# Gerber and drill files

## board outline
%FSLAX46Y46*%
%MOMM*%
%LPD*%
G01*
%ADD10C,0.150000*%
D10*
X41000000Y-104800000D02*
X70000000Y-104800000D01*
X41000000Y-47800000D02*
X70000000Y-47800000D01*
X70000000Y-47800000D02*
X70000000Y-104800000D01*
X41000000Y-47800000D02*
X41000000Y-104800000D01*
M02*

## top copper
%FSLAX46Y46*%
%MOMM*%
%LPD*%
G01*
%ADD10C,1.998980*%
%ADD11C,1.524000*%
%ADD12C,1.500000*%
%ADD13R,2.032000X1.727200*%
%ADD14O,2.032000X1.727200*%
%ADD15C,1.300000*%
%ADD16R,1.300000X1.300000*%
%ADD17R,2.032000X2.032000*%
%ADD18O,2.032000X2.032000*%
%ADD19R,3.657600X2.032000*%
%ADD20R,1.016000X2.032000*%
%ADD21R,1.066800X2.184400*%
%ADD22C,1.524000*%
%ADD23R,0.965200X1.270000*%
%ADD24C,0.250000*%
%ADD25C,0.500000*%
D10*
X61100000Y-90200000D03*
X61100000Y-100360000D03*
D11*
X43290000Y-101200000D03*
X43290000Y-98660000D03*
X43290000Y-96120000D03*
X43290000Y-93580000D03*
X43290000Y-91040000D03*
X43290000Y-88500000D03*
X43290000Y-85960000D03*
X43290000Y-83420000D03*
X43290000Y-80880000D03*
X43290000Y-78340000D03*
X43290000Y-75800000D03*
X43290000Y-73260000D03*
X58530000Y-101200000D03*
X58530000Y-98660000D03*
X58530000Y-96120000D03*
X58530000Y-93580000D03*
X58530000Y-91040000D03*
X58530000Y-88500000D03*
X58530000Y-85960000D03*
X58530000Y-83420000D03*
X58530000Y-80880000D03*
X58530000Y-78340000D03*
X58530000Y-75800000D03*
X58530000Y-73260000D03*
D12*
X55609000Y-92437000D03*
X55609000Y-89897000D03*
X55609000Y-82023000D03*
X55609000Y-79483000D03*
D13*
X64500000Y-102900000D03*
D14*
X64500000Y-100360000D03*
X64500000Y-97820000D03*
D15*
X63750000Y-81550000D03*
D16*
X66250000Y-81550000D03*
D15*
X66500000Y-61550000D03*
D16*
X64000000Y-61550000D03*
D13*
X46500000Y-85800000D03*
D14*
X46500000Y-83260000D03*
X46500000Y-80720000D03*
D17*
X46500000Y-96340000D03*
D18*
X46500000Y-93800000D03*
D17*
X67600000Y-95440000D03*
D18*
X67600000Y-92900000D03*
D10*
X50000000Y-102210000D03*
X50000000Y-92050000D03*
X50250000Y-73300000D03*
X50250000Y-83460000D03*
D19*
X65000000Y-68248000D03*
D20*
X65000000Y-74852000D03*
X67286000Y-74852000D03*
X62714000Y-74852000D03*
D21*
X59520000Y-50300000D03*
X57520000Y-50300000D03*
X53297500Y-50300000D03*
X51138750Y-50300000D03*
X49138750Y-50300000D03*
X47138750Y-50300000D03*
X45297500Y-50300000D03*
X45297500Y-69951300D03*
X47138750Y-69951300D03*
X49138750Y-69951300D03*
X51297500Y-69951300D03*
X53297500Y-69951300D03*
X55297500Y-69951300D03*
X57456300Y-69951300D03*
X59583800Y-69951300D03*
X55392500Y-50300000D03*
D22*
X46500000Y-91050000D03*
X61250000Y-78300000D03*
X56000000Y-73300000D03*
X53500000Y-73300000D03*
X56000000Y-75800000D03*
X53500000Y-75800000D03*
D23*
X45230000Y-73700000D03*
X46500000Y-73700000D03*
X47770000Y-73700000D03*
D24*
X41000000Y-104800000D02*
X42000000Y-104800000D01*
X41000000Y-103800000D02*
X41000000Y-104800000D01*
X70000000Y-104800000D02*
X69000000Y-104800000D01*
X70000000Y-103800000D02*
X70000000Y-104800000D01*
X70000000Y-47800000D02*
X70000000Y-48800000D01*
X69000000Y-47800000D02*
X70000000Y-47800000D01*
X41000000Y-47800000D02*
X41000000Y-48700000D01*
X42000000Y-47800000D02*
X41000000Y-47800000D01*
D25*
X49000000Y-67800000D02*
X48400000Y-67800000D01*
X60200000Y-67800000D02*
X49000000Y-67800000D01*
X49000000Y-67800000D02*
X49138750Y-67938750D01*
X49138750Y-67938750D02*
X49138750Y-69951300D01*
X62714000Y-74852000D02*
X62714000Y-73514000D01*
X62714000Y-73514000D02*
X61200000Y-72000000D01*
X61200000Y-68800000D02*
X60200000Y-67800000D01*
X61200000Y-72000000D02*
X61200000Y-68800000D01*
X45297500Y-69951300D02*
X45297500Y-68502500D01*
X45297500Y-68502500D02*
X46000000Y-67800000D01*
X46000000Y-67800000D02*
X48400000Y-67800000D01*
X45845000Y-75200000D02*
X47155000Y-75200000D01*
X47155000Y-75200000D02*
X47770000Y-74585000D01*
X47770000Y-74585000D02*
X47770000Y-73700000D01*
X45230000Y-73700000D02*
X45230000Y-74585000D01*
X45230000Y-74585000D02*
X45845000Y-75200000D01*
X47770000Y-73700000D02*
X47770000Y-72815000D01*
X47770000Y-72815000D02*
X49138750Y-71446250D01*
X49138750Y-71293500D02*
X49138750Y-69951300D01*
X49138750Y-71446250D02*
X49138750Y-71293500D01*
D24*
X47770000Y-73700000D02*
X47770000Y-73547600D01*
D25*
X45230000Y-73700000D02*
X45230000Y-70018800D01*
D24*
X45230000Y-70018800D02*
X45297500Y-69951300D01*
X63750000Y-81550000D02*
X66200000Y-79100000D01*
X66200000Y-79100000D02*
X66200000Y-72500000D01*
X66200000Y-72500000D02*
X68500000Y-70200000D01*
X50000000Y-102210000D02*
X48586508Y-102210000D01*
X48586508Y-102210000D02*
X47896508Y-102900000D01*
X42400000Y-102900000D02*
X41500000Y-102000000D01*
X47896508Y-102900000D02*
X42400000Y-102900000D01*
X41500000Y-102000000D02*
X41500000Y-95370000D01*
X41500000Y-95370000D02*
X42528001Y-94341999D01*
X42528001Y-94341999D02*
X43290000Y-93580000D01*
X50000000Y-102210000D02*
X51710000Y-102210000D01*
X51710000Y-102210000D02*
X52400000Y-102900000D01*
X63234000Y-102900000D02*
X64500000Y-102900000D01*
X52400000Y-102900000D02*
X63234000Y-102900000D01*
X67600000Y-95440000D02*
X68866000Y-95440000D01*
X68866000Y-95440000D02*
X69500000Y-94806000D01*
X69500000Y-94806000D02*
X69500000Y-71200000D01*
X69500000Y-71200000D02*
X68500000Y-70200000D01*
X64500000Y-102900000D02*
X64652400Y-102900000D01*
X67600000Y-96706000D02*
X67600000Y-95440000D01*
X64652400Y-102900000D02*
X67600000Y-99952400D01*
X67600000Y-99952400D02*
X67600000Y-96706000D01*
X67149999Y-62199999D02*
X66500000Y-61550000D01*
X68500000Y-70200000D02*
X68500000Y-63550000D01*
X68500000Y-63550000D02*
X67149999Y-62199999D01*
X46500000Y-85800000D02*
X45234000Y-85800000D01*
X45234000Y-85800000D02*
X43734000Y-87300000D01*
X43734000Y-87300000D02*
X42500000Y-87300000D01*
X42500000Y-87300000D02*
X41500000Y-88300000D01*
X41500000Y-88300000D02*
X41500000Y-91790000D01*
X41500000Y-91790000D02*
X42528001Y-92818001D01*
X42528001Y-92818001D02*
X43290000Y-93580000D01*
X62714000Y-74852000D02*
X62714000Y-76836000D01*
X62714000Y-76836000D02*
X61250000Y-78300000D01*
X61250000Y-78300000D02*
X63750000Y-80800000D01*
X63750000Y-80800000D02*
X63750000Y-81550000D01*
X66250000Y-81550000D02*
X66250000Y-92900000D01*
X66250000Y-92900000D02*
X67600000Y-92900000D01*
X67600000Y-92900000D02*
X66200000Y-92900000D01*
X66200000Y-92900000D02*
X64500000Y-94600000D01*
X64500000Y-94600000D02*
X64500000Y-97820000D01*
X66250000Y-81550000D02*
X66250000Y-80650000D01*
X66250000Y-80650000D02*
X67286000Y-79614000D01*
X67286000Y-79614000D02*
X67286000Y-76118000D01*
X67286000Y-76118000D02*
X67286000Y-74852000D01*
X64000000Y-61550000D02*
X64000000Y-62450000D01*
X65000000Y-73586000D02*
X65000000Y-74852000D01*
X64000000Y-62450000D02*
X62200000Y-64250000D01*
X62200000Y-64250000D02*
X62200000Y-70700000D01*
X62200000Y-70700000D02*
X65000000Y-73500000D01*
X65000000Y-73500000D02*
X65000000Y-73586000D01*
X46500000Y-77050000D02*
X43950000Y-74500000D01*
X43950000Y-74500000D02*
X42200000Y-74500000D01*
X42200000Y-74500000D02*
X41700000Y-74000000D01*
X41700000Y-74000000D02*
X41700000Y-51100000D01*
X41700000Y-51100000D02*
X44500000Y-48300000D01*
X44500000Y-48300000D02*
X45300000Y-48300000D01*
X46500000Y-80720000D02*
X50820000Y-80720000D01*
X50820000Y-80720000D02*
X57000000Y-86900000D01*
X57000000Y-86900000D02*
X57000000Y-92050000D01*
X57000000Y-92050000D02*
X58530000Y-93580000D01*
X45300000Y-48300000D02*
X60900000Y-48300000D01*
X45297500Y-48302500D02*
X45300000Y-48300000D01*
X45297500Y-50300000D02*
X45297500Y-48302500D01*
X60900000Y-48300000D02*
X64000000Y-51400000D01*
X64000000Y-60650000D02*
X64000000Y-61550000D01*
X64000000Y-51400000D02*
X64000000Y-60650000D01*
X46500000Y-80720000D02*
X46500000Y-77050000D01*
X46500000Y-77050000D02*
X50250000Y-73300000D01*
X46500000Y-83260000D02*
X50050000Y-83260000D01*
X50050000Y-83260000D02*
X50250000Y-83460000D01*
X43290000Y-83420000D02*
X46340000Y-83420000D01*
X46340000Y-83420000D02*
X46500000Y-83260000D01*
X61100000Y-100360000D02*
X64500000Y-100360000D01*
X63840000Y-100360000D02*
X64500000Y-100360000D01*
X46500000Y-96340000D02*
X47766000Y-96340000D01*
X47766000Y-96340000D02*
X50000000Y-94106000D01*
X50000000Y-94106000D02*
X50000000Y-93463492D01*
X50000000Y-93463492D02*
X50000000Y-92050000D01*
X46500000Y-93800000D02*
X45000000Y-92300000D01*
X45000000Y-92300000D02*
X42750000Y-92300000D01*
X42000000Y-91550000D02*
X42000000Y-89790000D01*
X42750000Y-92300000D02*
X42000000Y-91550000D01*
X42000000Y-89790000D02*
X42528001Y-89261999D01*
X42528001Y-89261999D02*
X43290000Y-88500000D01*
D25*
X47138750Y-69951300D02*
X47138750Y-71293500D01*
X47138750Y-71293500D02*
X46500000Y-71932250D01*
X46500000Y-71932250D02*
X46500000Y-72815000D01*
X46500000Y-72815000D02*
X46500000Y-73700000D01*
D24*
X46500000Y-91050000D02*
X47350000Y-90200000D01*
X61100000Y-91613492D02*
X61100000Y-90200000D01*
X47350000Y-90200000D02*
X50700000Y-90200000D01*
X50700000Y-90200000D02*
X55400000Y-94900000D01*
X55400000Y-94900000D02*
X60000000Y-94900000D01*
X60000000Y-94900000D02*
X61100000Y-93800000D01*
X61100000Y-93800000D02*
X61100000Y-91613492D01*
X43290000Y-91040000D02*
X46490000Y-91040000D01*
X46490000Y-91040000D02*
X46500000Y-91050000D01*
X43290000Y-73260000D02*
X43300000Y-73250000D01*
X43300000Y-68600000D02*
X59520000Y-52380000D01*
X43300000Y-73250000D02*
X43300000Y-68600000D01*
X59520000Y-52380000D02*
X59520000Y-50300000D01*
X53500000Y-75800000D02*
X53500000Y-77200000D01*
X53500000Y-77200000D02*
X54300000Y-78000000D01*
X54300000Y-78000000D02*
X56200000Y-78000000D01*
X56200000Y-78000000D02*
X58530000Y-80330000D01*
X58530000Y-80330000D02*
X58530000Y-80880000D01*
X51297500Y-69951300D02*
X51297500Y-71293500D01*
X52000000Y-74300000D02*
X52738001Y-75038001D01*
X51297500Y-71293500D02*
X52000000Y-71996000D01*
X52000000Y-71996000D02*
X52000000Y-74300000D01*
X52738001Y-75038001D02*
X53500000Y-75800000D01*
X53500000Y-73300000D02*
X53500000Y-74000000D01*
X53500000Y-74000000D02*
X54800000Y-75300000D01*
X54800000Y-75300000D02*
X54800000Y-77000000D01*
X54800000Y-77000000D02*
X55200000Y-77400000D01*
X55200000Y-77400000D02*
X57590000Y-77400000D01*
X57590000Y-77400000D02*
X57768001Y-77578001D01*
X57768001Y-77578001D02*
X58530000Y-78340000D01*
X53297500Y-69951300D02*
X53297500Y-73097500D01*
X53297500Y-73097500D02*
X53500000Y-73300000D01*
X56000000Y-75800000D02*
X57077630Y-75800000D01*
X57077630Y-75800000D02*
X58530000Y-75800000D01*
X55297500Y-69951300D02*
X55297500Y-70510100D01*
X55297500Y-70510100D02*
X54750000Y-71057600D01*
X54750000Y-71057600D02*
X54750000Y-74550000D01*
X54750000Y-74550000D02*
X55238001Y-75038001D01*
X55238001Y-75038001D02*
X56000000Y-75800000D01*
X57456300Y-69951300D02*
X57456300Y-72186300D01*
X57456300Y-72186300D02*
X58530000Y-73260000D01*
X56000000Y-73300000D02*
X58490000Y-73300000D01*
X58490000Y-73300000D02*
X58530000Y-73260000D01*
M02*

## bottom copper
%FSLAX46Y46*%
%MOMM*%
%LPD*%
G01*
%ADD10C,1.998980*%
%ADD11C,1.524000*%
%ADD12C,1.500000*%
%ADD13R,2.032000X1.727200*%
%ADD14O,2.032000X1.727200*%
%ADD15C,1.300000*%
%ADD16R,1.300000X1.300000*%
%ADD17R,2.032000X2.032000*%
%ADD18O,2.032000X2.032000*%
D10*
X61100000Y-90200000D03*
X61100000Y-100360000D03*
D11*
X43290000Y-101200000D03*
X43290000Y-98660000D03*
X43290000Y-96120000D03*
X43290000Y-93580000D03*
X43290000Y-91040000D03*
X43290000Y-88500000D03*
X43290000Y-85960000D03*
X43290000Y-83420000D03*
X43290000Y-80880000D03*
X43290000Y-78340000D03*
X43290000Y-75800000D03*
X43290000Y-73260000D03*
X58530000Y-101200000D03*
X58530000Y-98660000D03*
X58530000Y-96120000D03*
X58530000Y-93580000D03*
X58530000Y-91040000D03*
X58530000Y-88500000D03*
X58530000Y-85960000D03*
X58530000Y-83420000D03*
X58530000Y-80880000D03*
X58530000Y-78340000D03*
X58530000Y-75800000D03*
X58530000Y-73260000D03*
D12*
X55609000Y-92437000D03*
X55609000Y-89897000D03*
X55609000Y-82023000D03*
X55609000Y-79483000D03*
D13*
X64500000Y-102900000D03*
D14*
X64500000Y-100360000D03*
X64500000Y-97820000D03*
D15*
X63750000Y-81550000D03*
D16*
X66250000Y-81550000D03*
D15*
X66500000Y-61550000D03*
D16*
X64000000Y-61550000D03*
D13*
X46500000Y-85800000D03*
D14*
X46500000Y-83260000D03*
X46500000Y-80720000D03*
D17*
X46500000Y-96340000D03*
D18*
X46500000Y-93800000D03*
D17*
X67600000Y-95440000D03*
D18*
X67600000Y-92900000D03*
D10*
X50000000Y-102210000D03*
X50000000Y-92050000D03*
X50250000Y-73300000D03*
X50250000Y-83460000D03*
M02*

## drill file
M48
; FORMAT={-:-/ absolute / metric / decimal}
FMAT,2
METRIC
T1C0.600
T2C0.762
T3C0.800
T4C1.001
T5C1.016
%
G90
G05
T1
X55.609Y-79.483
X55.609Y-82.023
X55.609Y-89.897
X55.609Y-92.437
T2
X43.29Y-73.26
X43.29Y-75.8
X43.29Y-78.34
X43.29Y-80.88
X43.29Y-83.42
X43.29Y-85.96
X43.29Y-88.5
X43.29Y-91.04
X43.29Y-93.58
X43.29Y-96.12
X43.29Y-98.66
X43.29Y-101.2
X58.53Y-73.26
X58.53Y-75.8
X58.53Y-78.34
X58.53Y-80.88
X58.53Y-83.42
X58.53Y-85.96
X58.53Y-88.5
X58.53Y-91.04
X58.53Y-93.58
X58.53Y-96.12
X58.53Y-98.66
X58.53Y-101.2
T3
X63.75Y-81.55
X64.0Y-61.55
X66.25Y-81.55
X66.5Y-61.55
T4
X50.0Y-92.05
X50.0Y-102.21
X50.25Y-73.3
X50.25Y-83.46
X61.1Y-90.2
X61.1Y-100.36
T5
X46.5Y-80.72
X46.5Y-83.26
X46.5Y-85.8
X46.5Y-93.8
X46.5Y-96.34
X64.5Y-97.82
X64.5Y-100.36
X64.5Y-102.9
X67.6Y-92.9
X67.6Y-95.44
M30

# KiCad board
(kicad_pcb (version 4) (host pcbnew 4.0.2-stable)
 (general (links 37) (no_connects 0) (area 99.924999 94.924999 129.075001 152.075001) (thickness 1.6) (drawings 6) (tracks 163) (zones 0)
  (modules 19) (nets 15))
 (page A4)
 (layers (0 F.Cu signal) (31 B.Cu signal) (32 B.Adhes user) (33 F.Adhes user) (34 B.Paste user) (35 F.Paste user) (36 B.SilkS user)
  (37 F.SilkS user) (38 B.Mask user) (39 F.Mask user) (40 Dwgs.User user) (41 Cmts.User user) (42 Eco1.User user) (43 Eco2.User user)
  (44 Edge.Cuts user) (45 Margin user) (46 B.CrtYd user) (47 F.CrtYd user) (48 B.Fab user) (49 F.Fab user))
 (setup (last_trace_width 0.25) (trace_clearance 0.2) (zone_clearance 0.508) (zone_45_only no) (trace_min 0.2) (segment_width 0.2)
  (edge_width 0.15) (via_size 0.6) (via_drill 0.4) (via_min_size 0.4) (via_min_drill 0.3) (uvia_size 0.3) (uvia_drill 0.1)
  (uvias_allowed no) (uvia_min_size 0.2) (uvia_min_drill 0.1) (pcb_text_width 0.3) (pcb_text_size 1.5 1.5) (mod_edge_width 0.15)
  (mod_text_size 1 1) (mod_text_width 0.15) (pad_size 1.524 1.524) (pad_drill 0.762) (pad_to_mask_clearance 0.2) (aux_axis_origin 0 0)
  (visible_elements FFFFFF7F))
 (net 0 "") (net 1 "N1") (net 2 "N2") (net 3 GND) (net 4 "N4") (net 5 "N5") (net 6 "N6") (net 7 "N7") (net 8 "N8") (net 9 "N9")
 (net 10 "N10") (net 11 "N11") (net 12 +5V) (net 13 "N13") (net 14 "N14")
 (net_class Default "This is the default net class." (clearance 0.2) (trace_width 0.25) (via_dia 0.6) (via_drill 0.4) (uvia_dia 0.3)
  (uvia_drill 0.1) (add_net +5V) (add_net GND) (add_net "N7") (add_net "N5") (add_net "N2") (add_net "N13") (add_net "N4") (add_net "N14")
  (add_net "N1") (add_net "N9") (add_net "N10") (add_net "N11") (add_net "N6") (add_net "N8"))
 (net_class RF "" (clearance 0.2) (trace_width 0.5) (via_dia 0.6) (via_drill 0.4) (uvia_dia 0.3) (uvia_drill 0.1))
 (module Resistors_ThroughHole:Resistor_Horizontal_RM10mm (layer F.Cu) (at 61.1 90.2 270)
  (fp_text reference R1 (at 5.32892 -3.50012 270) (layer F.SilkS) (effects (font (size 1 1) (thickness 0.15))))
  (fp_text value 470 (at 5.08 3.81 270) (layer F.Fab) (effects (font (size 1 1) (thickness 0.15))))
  (pad 1 thru_hole circle (at 0 0 270) (size 1.99898 1.99898) (drill 1.00076) (layers *.Cu *.SilkS *.Mask) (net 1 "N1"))
  (pad 2 thru_hole circle (at 10.16 0 270) (size 1.99898 1.99898) (drill 1.00076) (layers *.Cu *.SilkS *.Mask) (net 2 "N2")))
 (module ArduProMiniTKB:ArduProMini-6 (layer B.Cu) (at 40.75 107.55)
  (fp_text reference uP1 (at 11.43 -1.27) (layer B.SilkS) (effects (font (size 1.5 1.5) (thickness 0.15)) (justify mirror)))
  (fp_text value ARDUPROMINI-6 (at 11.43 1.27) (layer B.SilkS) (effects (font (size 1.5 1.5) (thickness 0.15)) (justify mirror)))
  (pad 7 thru_hole circle (at 2.54 -6.35) (size 1.524 1.524) (drill 0.762) (layers *.Cu *.Mask B.SilkS))
  (pad 8 thru_hole circle (at 2.54 -8.89) (size 1.524 1.524) (drill 0.762) (layers *.Cu *.Mask B.SilkS))
  (pad 9 thru_hole circle (at 2.54 -11.43) (size 1.524 1.524) (drill 0.762) (layers *.Cu *.Mask B.SilkS))
  (pad 10 thru_hole circle (at 2.54 -13.97) (size 1.524 1.524) (drill 0.762) (layers *.Cu *.Mask B.SilkS) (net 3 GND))
  (pad 11 thru_hole circle (at 2.54 -16.51) (size 1.524 1.524) (drill 0.762) (layers *.Cu *.Mask B.SilkS) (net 1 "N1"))
  (pad 12 thru_hole circle (at 2.54 -19.05) (size 1.524 1.524) (drill 0.762) (layers *.Cu *.Mask B.SilkS) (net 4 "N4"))
  (pad 13 thru_hole circle (at 2.54 -21.59) (size 1.524 1.524) (drill 0.762) (layers *.Cu *.Mask B.SilkS))
  (pad 14 thru_hole circle (at 2.54 -24.13) (size 1.524 1.524) (drill 0.762) (layers *.Cu *.Mask B.SilkS) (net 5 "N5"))
  (pad 15 thru_hole circle (at 2.54 -26.67) (size 1.524 1.524) (drill 0.762) (layers *.Cu *.Mask B.SilkS))
  (pad 16 thru_hole circle (at 2.54 -29.21) (size 1.524 1.524) (drill 0.762) (layers *.Cu *.Mask B.SilkS))
  (pad 17 thru_hole circle (at 2.54 -31.75) (size 1.524 1.524) (drill 0.762) (layers *.Cu *.Mask B.SilkS))
  (pad 18 thru_hole circle (at 2.54 -34.29) (size 1.524 1.524) (drill 0.762) (layers *.Cu *.Mask B.SilkS) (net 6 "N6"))
  (pad 19 thru_hole circle (at 17.78 -6.35) (size 1.524 1.524) (drill 0.762) (layers *.Cu *.Mask B.SilkS))
  (pad 20 thru_hole circle (at 17.78 -8.89) (size 1.524 1.524) (drill 0.762) (layers *.Cu *.Mask B.SilkS))
  (pad 21 thru_hole circle (at 17.78 -11.43) (size 1.524 1.524) (drill 0.762) (layers *.Cu *.Mask B.SilkS))
  (pad 22 thru_hole circle (at 17.78 -13.97) (size 1.524 1.524) (drill 0.762) (layers *.Cu *.Mask B.SilkS) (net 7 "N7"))
  (pad 23 thru_hole circle (at 17.78 -16.51) (size 1.524 1.524) (drill 0.762) (layers *.Cu *.Mask B.SilkS))
  (pad 24 thru_hole circle (at 17.78 -19.05) (size 1.524 1.524) (drill 0.762) (layers *.Cu *.Mask B.SilkS))
  (pad 25 thru_hole circle (at 17.78 -21.59) (size 1.524 1.524) (drill 0.762) (layers *.Cu *.Mask B.SilkS))
  (pad 26 thru_hole circle (at 17.78 -24.13) (size 1.524 1.524) (drill 0.762) (layers *.Cu *.Mask B.SilkS))
  (pad 27 thru_hole circle (at 17.78 -26.67) (size 1.524 1.524) (drill 0.762) (layers *.Cu *.Mask B.SilkS) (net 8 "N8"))
  (pad 28 thru_hole circle (at 17.78 -29.21) (size 1.524 1.524) (drill 0.762) (layers *.Cu *.Mask B.SilkS) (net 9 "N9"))
  (pad 29 thru_hole circle (at 17.78 -31.75) (size 1.524 1.524) (drill 0.762) (layers *.Cu *.Mask B.SilkS) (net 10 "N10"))
  (pad 30 thru_hole circle (at 17.78 -34.29) (size 1.524 1.524) (drill 0.762) (layers *.Cu *.Mask B.SilkS) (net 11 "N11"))
  (pad 31 thru_hole circle (at 14.859 -15.113) (size 1.5 1.5) (drill 0.6) (layers *.Cu *.Mask B.SilkS))
  (pad 32 thru_hole circle (at 14.859 -17.653) (size 1.5 1.5) (drill 0.6) (layers *.Cu *.Mask B.SilkS))
  (pad 34 thru_hole circle (at 14.859 -25.527) (size 1.5 1.5) (drill 0.6) (layers *.Cu *.Mask B.SilkS))
  (pad 35 thru_hole circle (at 14.859 -28.067) (size 1.5 1.5) (drill 0.6) (layers *.Cu *.Mask B.SilkS)))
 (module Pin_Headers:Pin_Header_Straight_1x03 (layer F.Cu) (at 64.5 102.9 180)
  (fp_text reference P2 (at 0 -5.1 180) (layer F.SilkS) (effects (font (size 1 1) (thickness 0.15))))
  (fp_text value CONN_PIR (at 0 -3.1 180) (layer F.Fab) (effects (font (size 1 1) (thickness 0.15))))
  (pad 1 thru_hole rect (at 0 0 180) (size 2.032 1.7272) (drill 1.016) (layers *.Cu *.Mask F.SilkS) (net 3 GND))
  (pad 2 thru_hole oval (at 0 2.54 180) (size 2.032 1.7272) (drill 1.016) (layers *.Cu *.Mask F.SilkS) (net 2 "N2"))
  (pad 3 thru_hole oval (at 0 5.08 180) (size 2.032 1.7272) (drill 1.016) (layers *.Cu *.Mask F.SilkS) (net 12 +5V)))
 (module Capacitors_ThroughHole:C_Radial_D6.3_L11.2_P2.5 (layer F.Cu) (at 66.25 81.55 180)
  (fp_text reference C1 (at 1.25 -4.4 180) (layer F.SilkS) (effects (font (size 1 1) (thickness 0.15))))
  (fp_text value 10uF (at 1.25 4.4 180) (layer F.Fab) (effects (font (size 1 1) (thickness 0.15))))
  (pad 2 thru_hole circle (at 2.5 0 180) (size 1.3 1.3) (drill 0.8) (layers *.Cu *.Mask F.SilkS) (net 3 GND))
  (pad 1 thru_hole rect (at 0 0 180) (size 1.3 1.3) (drill 0.8) (layers *.Cu *.Mask F.SilkS) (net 12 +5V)))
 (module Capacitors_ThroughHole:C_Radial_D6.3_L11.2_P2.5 (layer F.Cu) (at 64 61.55)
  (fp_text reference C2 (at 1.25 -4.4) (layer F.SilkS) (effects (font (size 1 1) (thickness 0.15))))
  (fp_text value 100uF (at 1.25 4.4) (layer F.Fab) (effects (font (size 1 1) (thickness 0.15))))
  (pad 2 thru_hole circle (at 2.5 0) (size 1.3 1.3) (drill 0.8) (layers *.Cu *.Mask F.SilkS) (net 3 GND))
  (pad 1 thru_hole rect (at 0 0) (size 1.3 1.3) (drill 0.8) (layers *.Cu *.Mask F.SilkS) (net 7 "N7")))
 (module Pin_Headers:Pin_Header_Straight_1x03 (layer F.Cu) (at 46.5 85.8 180)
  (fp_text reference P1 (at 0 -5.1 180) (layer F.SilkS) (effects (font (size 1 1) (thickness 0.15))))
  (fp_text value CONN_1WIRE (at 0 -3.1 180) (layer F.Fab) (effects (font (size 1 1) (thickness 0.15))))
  (pad 1 thru_hole rect (at 0 0 180) (size 2.032 1.7272) (drill 1.016) (layers *.Cu *.Mask F.SilkS) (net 3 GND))
  (pad 2 thru_hole oval (at 0 2.54 180) (size 2.032 1.7272) (drill 1.016) (layers *.Cu *.Mask F.SilkS) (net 5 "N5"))
  (pad 3 thru_hole oval (at 0 5.08 180) (size 2.032 1.7272) (drill 1.016) (layers *.Cu *.Mask F.SilkS) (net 7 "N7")))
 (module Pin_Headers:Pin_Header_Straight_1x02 (layer F.Cu) (at 46.5 96.34 180)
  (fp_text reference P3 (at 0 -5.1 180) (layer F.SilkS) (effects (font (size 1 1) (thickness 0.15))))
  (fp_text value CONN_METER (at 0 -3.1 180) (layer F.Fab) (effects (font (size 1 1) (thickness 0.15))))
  (pad 1 thru_hole rect (at 0 0 180) (size 2.032 2.032) (drill 1.016) (layers *.Cu *.Mask F.SilkS) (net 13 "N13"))
  (pad 2 thru_hole oval (at 0 2.54 180) (size 2.032 2.032) (drill 1.016) (layers *.Cu *.Mask F.SilkS) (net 4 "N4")))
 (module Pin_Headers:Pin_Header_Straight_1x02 (layer F.Cu) (at 67.6 95.44 180)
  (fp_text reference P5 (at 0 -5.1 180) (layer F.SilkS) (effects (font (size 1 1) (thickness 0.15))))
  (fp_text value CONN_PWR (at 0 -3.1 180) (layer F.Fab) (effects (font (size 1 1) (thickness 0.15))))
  (pad 1 thru_hole rect (at 0 0 180) (size 2.032 2.032) (drill 1.016) (layers *.Cu *.Mask F.SilkS) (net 3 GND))
  (pad 2 thru_hole oval (at 0 2.54 180) (size 2.032 2.032) (drill 1.016) (layers *.Cu *.Mask F.SilkS) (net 12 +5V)))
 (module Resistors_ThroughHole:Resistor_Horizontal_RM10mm (layer F.Cu) (at 50 102.21 90)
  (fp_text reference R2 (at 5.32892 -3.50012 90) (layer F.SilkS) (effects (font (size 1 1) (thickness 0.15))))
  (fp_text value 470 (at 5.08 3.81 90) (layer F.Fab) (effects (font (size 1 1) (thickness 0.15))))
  (pad 1 thru_hole circle (at 0 0 90) (size 1.99898 1.99898) (drill 1.00076) (layers *.Cu *.SilkS *.Mask) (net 3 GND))
  (pad 2 thru_hole circle (at 10.16 0 90) (size 1.99898 1.99898) (drill 1.00076) (layers *.Cu *.SilkS *.Mask) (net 13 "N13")))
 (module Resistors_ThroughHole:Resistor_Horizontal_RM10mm (layer F.Cu) (at 50.25 73.3 270)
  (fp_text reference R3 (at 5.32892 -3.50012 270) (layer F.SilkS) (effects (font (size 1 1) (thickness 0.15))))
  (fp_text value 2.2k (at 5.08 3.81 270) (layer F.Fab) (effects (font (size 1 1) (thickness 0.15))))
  (pad 1 thru_hole circle (at 0 0 270) (size 1.99898 1.99898) (drill 1.00076) (layers *.Cu *.SilkS *.Mask) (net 7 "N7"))
  (pad 2 thru_hole circle (at 10.16 0 270) (size 1.99898 1.99898) (drill 1.00076) (layers *.Cu *.SilkS *.Mask) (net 5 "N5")))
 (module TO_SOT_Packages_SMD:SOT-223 (layer F.Cu) (at 65 71.55)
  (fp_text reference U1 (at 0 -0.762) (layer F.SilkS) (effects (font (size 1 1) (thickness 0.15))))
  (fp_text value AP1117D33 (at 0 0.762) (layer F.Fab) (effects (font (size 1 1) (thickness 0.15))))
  (pad 4 smd rect (at 0 -3.302) (size 3.6576 2.032) (layers F.Cu F.Paste F.Mask))
  (pad 2 smd rect (at 0 3.302) (size 1.016 2.032) (layers F.Cu F.Paste F.Mask) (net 7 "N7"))
  (pad 3 smd rect (at 2.286 3.302) (size 1.016 2.032) (layers F.Cu F.Paste F.Mask) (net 12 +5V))
  (pad 1 smd rect (at -2.286 3.302) (size 1.016 2.032) (layers F.Cu F.Paste F.Mask) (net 3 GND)))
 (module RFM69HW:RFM (layer F.Cu) (at 44.25 50.3 270) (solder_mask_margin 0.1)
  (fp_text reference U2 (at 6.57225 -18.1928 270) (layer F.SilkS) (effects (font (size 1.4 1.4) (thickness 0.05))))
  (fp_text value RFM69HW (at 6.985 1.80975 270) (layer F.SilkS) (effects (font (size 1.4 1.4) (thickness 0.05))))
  (pad RESE smd rect (at 0 -15.27 270) (size 2.1844 1.0668) (layers F.Cu F.Paste F.Mask) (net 6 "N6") (solder_mask_margin 0.2))
  (pad DIO0 smd rect (at 0 -13.27 270) (size 2.1844 1.0668) (layers F.Cu F.Paste F.Mask) (solder_mask_margin 0.2))
  (pad DIO2 smd rect (at 0 -9.0475 270) (size 2.1844 1.0668) (layers F.Cu F.Paste F.Mask) (solder_mask_margin 0.2))
  (pad DIO3 smd rect (at 0 -6.88875 270) (size 2.1844 1.0668) (layers F.Cu F.Paste F.Mask) (solder_mask_margin 0.2))
  (pad DIO4 smd rect (at 0 -4.88875 270) (size 2.1844 1.0668) (layers F.Cu F.Paste F.Mask) (solder_mask_margin 0.2))
  (pad DIO5 smd rect (at 0 -2.88875 270) (size 2.1844 1.0668) (layers F.Cu F.Paste F.Mask) (solder_mask_margin 0.2))
  (pad VCC smd rect (at 0 -1.0475 270) (size 2.1844 1.0668) (layers F.Cu F.Paste F.Mask) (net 7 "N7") (solder_mask_margin 0.2))
  (pad GNDB smd rect (at 19.6513 -1.0475 270) (size 2.1844 1.0668) (layers F.Cu F.Paste F.Mask) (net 3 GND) (solder_mask_margin 0.2))
  (pad ANT smd rect (at 19.6513 -2.88875 270) (size 2.1844 1.0668) (layers F.Cu F.Paste F.Mask) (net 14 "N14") (solder_mask_margin 0.2))
  (pad GNDA smd rect (at 19.6513 -4.88875 270) (size 2.1844 1.0668) (layers F.Cu F.Paste F.Mask) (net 3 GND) (solder_mask_margin 0.2))
  (pad SCK smd rect (at 19.6513 -7.0475 270) (size 2.1844 1.0668) (layers F.Cu F.Paste F.Mask) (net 8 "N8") (solder_mask_margin 0.2))
  (pad MISO smd rect (at 19.6513 -9.0475 270) (size 2.1844 1.0668) (layers F.Cu F.Paste F.Mask) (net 9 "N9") (solder_mask_margin 0.2))
  (pad MOSI smd rect (at 19.6513 -11.0475 270) (size 2.1844 1.0668) (layers F.Cu F.Paste F.Mask) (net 10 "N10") (solder_mask_margin 0.2))
  (pad NSS smd rect (at 19.6513 -13.2063 270) (size 2.1844 1.0668) (layers F.Cu F.Paste F.Mask) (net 11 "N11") (solder_mask_margin 0.2))
  (pad NC smd rect (at 19.6513 -15.3338 270) (size 2.1844 1.0668) (layers F.Cu F.Paste F.Mask) (solder_mask_margin 0.2))
  (pad DIO1 smd rect (at 0 -11.1425 270) (size 2.1844 1.0668) (layers F.Cu F.Paste F.Mask) (solder_mask_margin 0.2)))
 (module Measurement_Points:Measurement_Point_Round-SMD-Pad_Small (layer F.Cu) (at 46.5 91.05)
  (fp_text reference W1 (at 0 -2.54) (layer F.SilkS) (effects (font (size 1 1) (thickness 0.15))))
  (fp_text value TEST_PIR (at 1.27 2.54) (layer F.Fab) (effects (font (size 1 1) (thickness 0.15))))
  (pad 1 smd circle (at 0 0) (size 1.524 1.524) (layers F.Cu F.Paste F.Mask) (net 1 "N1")))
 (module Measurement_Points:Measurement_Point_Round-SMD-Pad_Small (layer F.Cu) (at 61.25 78.3)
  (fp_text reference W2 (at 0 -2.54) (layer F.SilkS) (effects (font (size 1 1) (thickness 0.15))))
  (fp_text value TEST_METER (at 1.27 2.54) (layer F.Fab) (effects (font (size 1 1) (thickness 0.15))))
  (pad 1 smd circle (at 0 0) (size 1.524 1.524) (layers F.Cu F.Paste F.Mask) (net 3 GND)))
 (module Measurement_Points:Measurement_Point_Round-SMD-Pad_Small (layer F.Cu) (at 56 73.3)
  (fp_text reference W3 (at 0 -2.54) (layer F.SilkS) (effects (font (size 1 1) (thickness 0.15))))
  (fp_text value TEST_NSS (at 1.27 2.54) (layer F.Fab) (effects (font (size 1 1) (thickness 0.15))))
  (pad 1 smd circle (at 0 0) (size 1.524 1.524) (layers F.Cu F.Paste F.Mask) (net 11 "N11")))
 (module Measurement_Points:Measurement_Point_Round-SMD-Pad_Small (layer F.Cu) (at 53.5 73.3)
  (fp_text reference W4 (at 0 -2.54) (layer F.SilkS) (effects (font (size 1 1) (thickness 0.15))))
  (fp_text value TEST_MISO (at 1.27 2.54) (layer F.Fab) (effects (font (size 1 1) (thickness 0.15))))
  (pad 1 smd circle (at 0 0) (size 1.524 1.524) (layers F.Cu F.Paste F.Mask) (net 9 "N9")))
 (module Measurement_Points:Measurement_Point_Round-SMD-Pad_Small (layer F.Cu) (at 56 75.8)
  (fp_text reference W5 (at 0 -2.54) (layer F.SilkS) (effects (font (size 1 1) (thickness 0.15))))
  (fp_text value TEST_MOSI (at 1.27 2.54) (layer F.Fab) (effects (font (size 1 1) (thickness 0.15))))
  (pad 1 smd circle (at 0 0) (size 1.524 1.524) (layers F.Cu F.Paste F.Mask) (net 10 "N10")))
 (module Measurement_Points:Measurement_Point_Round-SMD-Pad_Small (layer F.Cu) (at 53.5 75.8)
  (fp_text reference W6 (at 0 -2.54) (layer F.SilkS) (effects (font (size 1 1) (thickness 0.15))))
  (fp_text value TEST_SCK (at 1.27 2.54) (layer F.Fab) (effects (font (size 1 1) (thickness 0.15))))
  (pad 1 smd circle (at 0 0) (size 1.524 1.524) (layers F.Cu F.Paste F.Mask) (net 8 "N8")))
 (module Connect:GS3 (layer F.Cu) (at 46.5 73.7 90)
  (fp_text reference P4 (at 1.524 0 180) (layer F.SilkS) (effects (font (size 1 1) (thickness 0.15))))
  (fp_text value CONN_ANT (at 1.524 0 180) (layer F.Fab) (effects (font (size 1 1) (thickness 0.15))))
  (pad 1 smd rect (at 0 -1.27 90) (size 1.27 0.9652) (layers F.Cu F.Paste F.Mask) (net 3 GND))
  (pad 2 smd rect (at 0 0 90) (size 1.27 0.9652) (layers F.Cu F.Paste F.Mask) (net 14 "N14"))
  (pad 3 smd rect (at 0 1.27 90) (size 1.27 0.9652) (layers F.Cu F.Paste F.Mask) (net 3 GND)))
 (gr_line (start 41 104.8) (end 70 104.8) (angle 90) (layer Edge.Cuts) (width 0.15))
 (gr_line (start 41 47.8) (end 70 47.8) (angle 90) (layer Edge.Cuts) (width 0.15))
 (gr_line (start 70 47.8) (end 70 104.8) (angle 90) (layer Edge.Cuts) (width 0.15))
 (gr_line (start 41 47.8) (end 41 104.8) (angle 90) (layer Edge.Cuts) (width 0.15))
 (segment (start 41 104.8) (end 42 104.8) (width 0.25) (layer F.Cu) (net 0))
 (segment (start 41 103.8) (end 41 104.8) (width 0.25) (layer F.Cu) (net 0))
 (segment (start 70 104.8) (end 69 104.8) (width 0.25) (layer F.Cu) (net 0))
 (segment (start 70 103.8) (end 70 104.8) (width 0.25) (layer F.Cu) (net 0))
 (segment (start 70 47.8) (end 70 48.8) (width 0.25) (layer F.Cu) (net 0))
 (segment (start 69 47.8) (end 70 47.8) (width 0.25) (layer F.Cu) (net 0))
 (segment (start 41 47.8) (end 41 48.7) (width 0.25) (layer F.Cu) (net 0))
 (segment (start 42 47.8) (end 41 47.8) (width 0.25) (layer F.Cu) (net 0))
 (segment (start 49 67.8) (end 48.4 67.8) (width 0.5) (layer F.Cu) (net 3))
 (segment (start 60.2 67.8) (end 49 67.8) (width 0.5) (layer F.Cu) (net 3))
 (segment (start 49 67.8) (end 49.13875 67.93875) (width 0.5) (layer F.Cu) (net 3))
 (segment (start 49.13875 67.93875) (end 49.13875 69.9513) (width 0.5) (layer F.Cu) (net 3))
 (segment (start 62.714 74.852) (end 62.714 73.514) (width 0.5) (layer F.Cu) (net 3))
 (segment (start 62.714 73.514) (end 61.2 72) (width 0.5) (layer F.Cu) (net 3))
 (segment (start 61.2 68.8) (end 60.2 67.8) (width 0.5) (layer F.Cu) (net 3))
 (segment (start 61.2 72) (end 61.2 68.8) (width 0.5) (layer F.Cu) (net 3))
 (segment (start 45.2975 69.9513) (end 45.2975 68.5025) (width 0.5) (layer F.Cu) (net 3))
 (segment (start 45.2975 68.5025) (end 46 67.8) (width 0.5) (layer F.Cu) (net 3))
 (segment (start 46 67.8) (end 48.4 67.8) (width 0.5) (layer F.Cu) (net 3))
 (segment (start 45.845 75.2) (end 47.155 75.2) (width 0.5) (layer F.Cu) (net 3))
 (segment (start 47.155 75.2) (end 47.77 74.585) (width 0.5) (layer F.Cu) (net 3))
 (segment (start 47.77 74.585) (end 47.77 73.7) (width 0.5) (layer F.Cu) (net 3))
 (segment (start 45.23 73.7) (end 45.23 74.585) (width 0.5) (layer F.Cu) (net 3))
 (segment (start 45.23 74.585) (end 45.845 75.2) (width 0.5) (layer F.Cu) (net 3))
 (segment (start 47.77 73.7) (end 47.77 72.815) (width 0.5) (layer F.Cu) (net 3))
 (segment (start 47.77 72.815) (end 49.13875 71.44625) (width 0.5) (layer F.Cu) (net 3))
 (segment (start 49.13875 71.2935) (end 49.13875 69.9513) (width 0.5) (layer F.Cu) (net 3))
 (segment (start 49.13875 71.44625) (end 49.13875 71.2935) (width 0.5) (layer F.Cu) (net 3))
 (segment (start 47.77 73.7) (end 47.77 73.5476) (width 0.25) (layer F.Cu) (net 3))
 (segment (start 45.23 73.7) (end 45.23 70.0188) (width 0.5) (layer F.Cu) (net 3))
 (segment (start 45.23 70.0188) (end 45.2975 69.9513) (width 0.25) (layer F.Cu) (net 3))
 (segment (start 63.75 81.55) (end 66.2 79.1) (width 0.25) (layer F.Cu) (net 3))
 (segment (start 66.2 79.1) (end 66.2 72.5) (width 0.25) (layer F.Cu) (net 3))
 (segment (start 66.2 72.5) (end 68.5 70.2) (width 0.25) (layer F.Cu) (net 3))
 (segment (start 50 102.21) (end 48.586508 102.21) (width 0.25) (layer F.Cu) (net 3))
 (segment (start 48.586508 102.21) (end 47.896508 102.9) (width 0.25) (layer F.Cu) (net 3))
 (segment (start 42.4 102.9) (end 41.5 102) (width 0.25) (layer F.Cu) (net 3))
 (segment (start 47.896508 102.9) (end 42.4 102.9) (width 0.25) (layer F.Cu) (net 3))
 (segment (start 41.5 102) (end 41.5 95.37) (width 0.25) (layer F.Cu) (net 3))
 (segment (start 41.5 95.37) (end 42.528001 94.341999) (width 0.25) (layer F.Cu) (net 3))
 (segment (start 42.528001 94.341999) (end 43.29 93.58) (width 0.25) (layer F.Cu) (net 3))
 (segment (start 50 102.21) (end 51.71 102.21) (width 0.25) (layer F.Cu) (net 3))
 (segment (start 51.71 102.21) (end 52.4 102.9) (width 0.25) (layer F.Cu) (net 3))
 (segment (start 63.234 102.9) (end 64.5 102.9) (width 0.25) (layer F.Cu) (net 3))
 (segment (start 52.4 102.9) (end 63.234 102.9) (width 0.25) (layer F.Cu) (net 3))
 (segment (start 67.6 95.44) (end 68.866 95.44) (width 0.25) (layer F.Cu) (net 3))
 (segment (start 68.866 95.44) (end 69.5 94.806) (width 0.25) (layer F.Cu) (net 3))
 (segment (start 69.5 94.806) (end 69.5 71.2) (width 0.25) (layer F.Cu) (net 3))
 (segment (start 69.5 71.2) (end 68.5 70.2) (width 0.25) (layer F.Cu) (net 3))
 (segment (start 64.5 102.9) (end 64.6524 102.9) (width 0.25) (layer F.Cu) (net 3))
 (segment (start 67.6 96.706) (end 67.6 95.44) (width 0.25) (layer F.Cu) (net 3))
 (segment (start 64.6524 102.9) (end 67.6 99.9524) (width 0.25) (layer F.Cu) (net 3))
 (segment (start 67.6 99.9524) (end 67.6 96.706) (width 0.25) (layer F.Cu) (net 3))
 (segment (start 67.149999 62.199999) (end 66.5 61.55) (width 0.25) (layer F.Cu) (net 3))
 (segment (start 68.5 70.2) (end 68.5 63.55) (width 0.25) (layer F.Cu) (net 3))
 (segment (start 68.5 63.55) (end 67.149999 62.199999) (width 0.25) (layer F.Cu) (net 3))
 (segment (start 46.5 85.8) (end 45.234 85.8) (width 0.25) (layer F.Cu) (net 3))
 (segment (start 45.234 85.8) (end 43.734 87.3) (width 0.25) (layer F.Cu) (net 3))
 (segment (start 43.734 87.3) (end 42.5 87.3) (width 0.25) (layer F.Cu) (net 3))
 (segment (start 42.5 87.3) (end 41.5 88.3) (width 0.25) (layer F.Cu) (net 3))
 (segment (start 41.5 88.3) (end 41.5 91.79) (width 0.25) (layer F.Cu) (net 3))
 (segment (start 41.5 91.79) (end 42.528001 92.818001) (width 0.25) (layer F.Cu) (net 3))
 (segment (start 42.528001 92.818001) (end 43.29 93.58) (width 0.25) (layer F.Cu) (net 3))
 (segment (start 62.714 74.852) (end 62.714 76.836) (width 0.25) (layer F.Cu) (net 3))
 (segment (start 62.714 76.836) (end 61.25 78.3) (width 0.25) (layer F.Cu) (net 3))
 (segment (start 61.25 78.3) (end 63.75 80.8) (width 0.25) (layer F.Cu) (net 3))
 (segment (start 63.75 80.8) (end 63.75 81.55) (width 0.25) (layer F.Cu) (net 3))
 (segment (start 66.25 81.55) (end 66.25 92.9) (width 0.25) (layer F.Cu) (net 12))
 (segment (start 66.25 92.9) (end 67.6 92.9) (width 0.25) (layer F.Cu) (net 12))
 (segment (start 67.6 92.9) (end 66.2 92.9) (width 0.25) (layer F.Cu) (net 12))
 (segment (start 66.2 92.9) (end 64.5 94.6) (width 0.25) (layer F.Cu) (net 12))
 (segment (start 64.5 94.6) (end 64.5 97.82) (width 0.25) (layer F.Cu) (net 12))
 (segment (start 66.25 81.55) (end 66.25 80.65) (width 0.25) (layer F.Cu) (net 12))
 (segment (start 66.25 80.65) (end 67.286 79.614) (width 0.25) (layer F.Cu) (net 12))
 (segment (start 67.286 79.614) (end 67.286 76.118) (width 0.25) (layer F.Cu) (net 12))
 (segment (start 67.286 76.118) (end 67.286 74.852) (width 0.25) (layer F.Cu) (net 12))
 (segment (start 64 61.55) (end 64 62.45) (width 0.25) (layer F.Cu) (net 7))
 (segment (start 65 73.586) (end 65 74.852) (width 0.25) (layer F.Cu) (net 7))
 (segment (start 64 62.45) (end 62.2 64.25) (width 0.25) (layer F.Cu) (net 7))
 (segment (start 62.2 64.25) (end 62.2 70.7) (width 0.25) (layer F.Cu) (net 7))
 (segment (start 62.2 70.7) (end 65 73.5) (width 0.25) (layer F.Cu) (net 7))
 (segment (start 65 73.5) (end 65 73.586) (width 0.25) (layer F.Cu) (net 7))
 (segment (start 46.5 77.05) (end 43.95 74.5) (width 0.25) (layer F.Cu) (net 7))
 (segment (start 43.95 74.5) (end 42.2 74.5) (width 0.25) (layer F.Cu) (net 7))
 (segment (start 42.2 74.5) (end 41.7 74) (width 0.25) (layer F.Cu) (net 7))
 (segment (start 41.7 74) (end 41.7 51.1) (width 0.25) (layer F.Cu) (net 7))
 (segment (start 41.7 51.1) (end 44.5 48.3) (width 0.25) (layer F.Cu) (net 7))
 (segment (start 44.5 48.3) (end 45.3 48.3) (width 0.25) (layer F.Cu) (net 7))
 (segment (start 46.5 80.72) (end 50.82 80.72) (width 0.25) (layer F.Cu) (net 7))
 (segment (start 50.82 80.72) (end 57 86.9) (width 0.25) (layer F.Cu) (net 7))
 (segment (start 57 86.9) (end 57 92.05) (width 0.25) (layer F.Cu) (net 7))
 (segment (start 57 92.05) (end 58.53 93.58) (width 0.25) (layer F.Cu) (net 7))
 (segment (start 45.3 48.3) (end 60.9 48.3) (width 0.25) (layer F.Cu) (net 7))
 (segment (start 45.2975 48.3025) (end 45.3 48.3) (width 0.25) (layer F.Cu) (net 7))
 (segment (start 45.2975 50.3) (end 45.2975 48.3025) (width 0.25) (layer F.Cu) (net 7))
 (segment (start 60.9 48.3) (end 64 51.4) (width 0.25) (layer F.Cu) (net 7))
 (segment (start 64 60.65) (end 64 61.55) (width 0.25) (layer F.Cu) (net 7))
 (segment (start 64 51.4) (end 64 60.65) (width 0.25) (layer F.Cu) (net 7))
 (segment (start 46.5 80.72) (end 46.5 77.05) (width 0.25) (layer F.Cu) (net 7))
 (segment (start 46.5 77.05) (end 50.25 73.3) (width 0.25) (layer F.Cu) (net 7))
 (segment (start 46.5 83.26) (end 50.05 83.26) (width 0.25) (layer F.Cu) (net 5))
 (segment (start 50.05 83.26) (end 50.25 83.46) (width 0.25) (layer F.Cu) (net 5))
 (segment (start 43.29 83.42) (end 46.34 83.42) (width 0.25) (layer F.Cu) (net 5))
 (segment (start 46.34 83.42) (end 46.5 83.26) (width 0.25) (layer F.Cu) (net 5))
 (segment (start 61.1 100.36) (end 64.5 100.36) (width 0.25) (layer F.Cu) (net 2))
 (segment (start 63.84 100.36) (end 64.5 100.36) (width 0.25) (layer F.Cu) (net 2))
 (segment (start 46.5 96.34) (end 47.766 96.34) (width 0.25) (layer F.Cu) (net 13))
 (segment (start 47.766 96.34) (end 50 94.106) (width 0.25) (layer F.Cu) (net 13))
 (segment (start 50 94.106) (end 50 93.463492) (width 0.25) (layer F.Cu) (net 13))
 (segment (start 50 93.463492) (end 50 92.05) (width 0.25) (layer F.Cu) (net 13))
 (segment (start 46.5 93.8) (end 45 92.3) (width 0.25) (layer F.Cu) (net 4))
 (segment (start 45 92.3) (end 42.75 92.3) (width 0.25) (layer F.Cu) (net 4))
 (segment (start 42 91.55) (end 42 89.79) (width 0.25) (layer F.Cu) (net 4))
 (segment (start 42.75 92.3) (end 42 91.55) (width 0.25) (layer F.Cu) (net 4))
 (segment (start 42 89.79) (end 42.528001 89.261999) (width 0.25) (layer F.Cu) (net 4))
 (segment (start 42.528001 89.261999) (end 43.29 88.5) (width 0.25) (layer F.Cu) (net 4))
 (segment (start 47.13875 69.9513) (end 47.13875 71.2935) (width 0.5) (layer F.Cu) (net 14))
 (segment (start 47.13875 71.2935) (end 46.5 71.93225) (width 0.5) (layer F.Cu) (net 14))
 (segment (start 46.5 71.93225) (end 46.5 72.815) (width 0.5) (layer F.Cu) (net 14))
 (segment (start 46.5 72.815) (end 46.5 73.7) (width 0.5) (layer F.Cu) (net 14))
 (segment (start 46.5 91.05) (end 47.35 90.2) (width 0.25) (layer F.Cu) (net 1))
 (segment (start 61.1 91.613492) (end 61.1 90.2) (width 0.25) (layer F.Cu) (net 1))
 (segment (start 47.35 90.2) (end 50.7 90.2) (width 0.25) (layer F.Cu) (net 1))
 (segment (start 50.7 90.2) (end 55.4 94.9) (width 0.25) (layer F.Cu) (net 1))
 (segment (start 55.4 94.9) (end 60 94.9) (width 0.25) (layer F.Cu) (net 1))
 (segment (start 60 94.9) (end 61.1 93.8) (width 0.25) (layer F.Cu) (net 1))
 (segment (start 61.1 93.8) (end 61.1 91.613492) (width 0.25) (layer F.Cu) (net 1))
 (segment (start 43.29 91.04) (end 46.49 91.04) (width 0.25) (layer F.Cu) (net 1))
 (segment (start 46.49 91.04) (end 46.5 91.05) (width 0.25) (layer F.Cu) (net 1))
 (segment (start 43.29 73.26) (end 43.3 73.25) (width 0.25) (layer F.Cu) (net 6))
 (segment (start 43.3 68.6) (end 59.52 52.38) (width 0.25) (layer F.Cu) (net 6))
 (segment (start 43.3 73.25) (end 43.3 68.6) (width 0.25) (layer F.Cu) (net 6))
 (segment (start 59.52 52.38) (end 59.52 50.3) (width 0.25) (layer F.Cu) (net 6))
 (segment (start 53.5 75.8) (end 53.5 77.2) (width 0.25) (layer F.Cu) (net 8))
 (segment (start 53.5 77.2) (end 54.3 78) (width 0.25) (layer F.Cu) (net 8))
 (segment (start 54.3 78) (end 56.2 78) (width 0.25) (layer F.Cu) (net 8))
 (segment (start 56.2 78) (end 58.53 80.33) (width 0.25) (layer F.Cu) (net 8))
 (segment (start 58.53 80.33) (end 58.53 80.88) (width 0.25) (layer F.Cu) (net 8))
 (segment (start 51.2975 69.9513) (end 51.2975 71.2935) (width 0.25) (layer F.Cu) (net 8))
 (segment (start 52 74.3) (end 52.738001 75.038001) (width 0.25) (layer F.Cu) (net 8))
 (segment (start 51.2975 71.2935) (end 52 71.996) (width 0.25) (layer F.Cu) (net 8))
 (segment (start 52 71.996) (end 52 74.3) (width 0.25) (layer F.Cu) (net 8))
 (segment (start 52.738001 75.038001) (end 53.5 75.8) (width 0.25) (layer F.Cu) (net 8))
 (segment (start 53.5 73.3) (end 53.5 74) (width 0.25) (layer F.Cu) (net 9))
 (segment (start 53.5 74) (end 54.8 75.3) (width 0.25) (layer F.Cu) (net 9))
 (segment (start 54.8 75.3) (end 54.8 77) (width 0.25) (layer F.Cu) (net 9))
 (segment (start 54.8 77) (end 55.2 77.4) (width 0.25) (layer F.Cu) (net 9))
 (segment (start 55.2 77.4) (end 57.59 77.4) (width 0.25) (layer F.Cu) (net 9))
 (segment (start 57.59 77.4) (end 57.768001 77.578001) (width 0.25) (layer F.Cu) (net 9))
 (segment (start 57.768001 77.578001) (end 58.53 78.34) (width 0.25) (layer F.Cu) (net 9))
 (segment (start 53.2975 69.9513) (end 53.2975 73.0975) (width 0.25) (layer F.Cu) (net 9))
 (segment (start 53.2975 73.0975) (end 53.5 73.3) (width 0.25) (layer F.Cu) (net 9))
 (segment (start 56 75.8) (end 57.07763 75.8) (width 0.25) (layer F.Cu) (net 10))
 (segment (start 57.07763 75.8) (end 58.53 75.8) (width 0.25) (layer F.Cu) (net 10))
 (segment (start 55.2975 69.9513) (end 55.2975 70.5101) (width 0.25) (layer F.Cu) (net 10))
 (segment (start 55.2975 70.5101) (end 54.75 71.0576) (width 0.25) (layer F.Cu) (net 10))
 (segment (start 54.75 71.0576) (end 54.75 74.55) (width 0.25) (layer F.Cu) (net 10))
 (segment (start 54.75 74.55) (end 55.238001 75.038001) (width 0.25) (layer F.Cu) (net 10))
 (segment (start 55.238001 75.038001) (end 56 75.8) (width 0.25) (layer F.Cu) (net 10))
 (segment (start 57.4563 69.9513) (end 57.4563 72.1863) (width 0.25) (layer F.Cu) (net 11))
 (segment (start 57.4563 72.1863) (end 58.53 73.26) (width 0.25) (layer F.Cu) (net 11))
 (segment (start 56 73.3) (end 58.49 73.3) (width 0.25) (layer F.Cu) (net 11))
 (segment (start 58.49 73.3) (end 58.53 73.26) (width 0.25) (layer F.Cu) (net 11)))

